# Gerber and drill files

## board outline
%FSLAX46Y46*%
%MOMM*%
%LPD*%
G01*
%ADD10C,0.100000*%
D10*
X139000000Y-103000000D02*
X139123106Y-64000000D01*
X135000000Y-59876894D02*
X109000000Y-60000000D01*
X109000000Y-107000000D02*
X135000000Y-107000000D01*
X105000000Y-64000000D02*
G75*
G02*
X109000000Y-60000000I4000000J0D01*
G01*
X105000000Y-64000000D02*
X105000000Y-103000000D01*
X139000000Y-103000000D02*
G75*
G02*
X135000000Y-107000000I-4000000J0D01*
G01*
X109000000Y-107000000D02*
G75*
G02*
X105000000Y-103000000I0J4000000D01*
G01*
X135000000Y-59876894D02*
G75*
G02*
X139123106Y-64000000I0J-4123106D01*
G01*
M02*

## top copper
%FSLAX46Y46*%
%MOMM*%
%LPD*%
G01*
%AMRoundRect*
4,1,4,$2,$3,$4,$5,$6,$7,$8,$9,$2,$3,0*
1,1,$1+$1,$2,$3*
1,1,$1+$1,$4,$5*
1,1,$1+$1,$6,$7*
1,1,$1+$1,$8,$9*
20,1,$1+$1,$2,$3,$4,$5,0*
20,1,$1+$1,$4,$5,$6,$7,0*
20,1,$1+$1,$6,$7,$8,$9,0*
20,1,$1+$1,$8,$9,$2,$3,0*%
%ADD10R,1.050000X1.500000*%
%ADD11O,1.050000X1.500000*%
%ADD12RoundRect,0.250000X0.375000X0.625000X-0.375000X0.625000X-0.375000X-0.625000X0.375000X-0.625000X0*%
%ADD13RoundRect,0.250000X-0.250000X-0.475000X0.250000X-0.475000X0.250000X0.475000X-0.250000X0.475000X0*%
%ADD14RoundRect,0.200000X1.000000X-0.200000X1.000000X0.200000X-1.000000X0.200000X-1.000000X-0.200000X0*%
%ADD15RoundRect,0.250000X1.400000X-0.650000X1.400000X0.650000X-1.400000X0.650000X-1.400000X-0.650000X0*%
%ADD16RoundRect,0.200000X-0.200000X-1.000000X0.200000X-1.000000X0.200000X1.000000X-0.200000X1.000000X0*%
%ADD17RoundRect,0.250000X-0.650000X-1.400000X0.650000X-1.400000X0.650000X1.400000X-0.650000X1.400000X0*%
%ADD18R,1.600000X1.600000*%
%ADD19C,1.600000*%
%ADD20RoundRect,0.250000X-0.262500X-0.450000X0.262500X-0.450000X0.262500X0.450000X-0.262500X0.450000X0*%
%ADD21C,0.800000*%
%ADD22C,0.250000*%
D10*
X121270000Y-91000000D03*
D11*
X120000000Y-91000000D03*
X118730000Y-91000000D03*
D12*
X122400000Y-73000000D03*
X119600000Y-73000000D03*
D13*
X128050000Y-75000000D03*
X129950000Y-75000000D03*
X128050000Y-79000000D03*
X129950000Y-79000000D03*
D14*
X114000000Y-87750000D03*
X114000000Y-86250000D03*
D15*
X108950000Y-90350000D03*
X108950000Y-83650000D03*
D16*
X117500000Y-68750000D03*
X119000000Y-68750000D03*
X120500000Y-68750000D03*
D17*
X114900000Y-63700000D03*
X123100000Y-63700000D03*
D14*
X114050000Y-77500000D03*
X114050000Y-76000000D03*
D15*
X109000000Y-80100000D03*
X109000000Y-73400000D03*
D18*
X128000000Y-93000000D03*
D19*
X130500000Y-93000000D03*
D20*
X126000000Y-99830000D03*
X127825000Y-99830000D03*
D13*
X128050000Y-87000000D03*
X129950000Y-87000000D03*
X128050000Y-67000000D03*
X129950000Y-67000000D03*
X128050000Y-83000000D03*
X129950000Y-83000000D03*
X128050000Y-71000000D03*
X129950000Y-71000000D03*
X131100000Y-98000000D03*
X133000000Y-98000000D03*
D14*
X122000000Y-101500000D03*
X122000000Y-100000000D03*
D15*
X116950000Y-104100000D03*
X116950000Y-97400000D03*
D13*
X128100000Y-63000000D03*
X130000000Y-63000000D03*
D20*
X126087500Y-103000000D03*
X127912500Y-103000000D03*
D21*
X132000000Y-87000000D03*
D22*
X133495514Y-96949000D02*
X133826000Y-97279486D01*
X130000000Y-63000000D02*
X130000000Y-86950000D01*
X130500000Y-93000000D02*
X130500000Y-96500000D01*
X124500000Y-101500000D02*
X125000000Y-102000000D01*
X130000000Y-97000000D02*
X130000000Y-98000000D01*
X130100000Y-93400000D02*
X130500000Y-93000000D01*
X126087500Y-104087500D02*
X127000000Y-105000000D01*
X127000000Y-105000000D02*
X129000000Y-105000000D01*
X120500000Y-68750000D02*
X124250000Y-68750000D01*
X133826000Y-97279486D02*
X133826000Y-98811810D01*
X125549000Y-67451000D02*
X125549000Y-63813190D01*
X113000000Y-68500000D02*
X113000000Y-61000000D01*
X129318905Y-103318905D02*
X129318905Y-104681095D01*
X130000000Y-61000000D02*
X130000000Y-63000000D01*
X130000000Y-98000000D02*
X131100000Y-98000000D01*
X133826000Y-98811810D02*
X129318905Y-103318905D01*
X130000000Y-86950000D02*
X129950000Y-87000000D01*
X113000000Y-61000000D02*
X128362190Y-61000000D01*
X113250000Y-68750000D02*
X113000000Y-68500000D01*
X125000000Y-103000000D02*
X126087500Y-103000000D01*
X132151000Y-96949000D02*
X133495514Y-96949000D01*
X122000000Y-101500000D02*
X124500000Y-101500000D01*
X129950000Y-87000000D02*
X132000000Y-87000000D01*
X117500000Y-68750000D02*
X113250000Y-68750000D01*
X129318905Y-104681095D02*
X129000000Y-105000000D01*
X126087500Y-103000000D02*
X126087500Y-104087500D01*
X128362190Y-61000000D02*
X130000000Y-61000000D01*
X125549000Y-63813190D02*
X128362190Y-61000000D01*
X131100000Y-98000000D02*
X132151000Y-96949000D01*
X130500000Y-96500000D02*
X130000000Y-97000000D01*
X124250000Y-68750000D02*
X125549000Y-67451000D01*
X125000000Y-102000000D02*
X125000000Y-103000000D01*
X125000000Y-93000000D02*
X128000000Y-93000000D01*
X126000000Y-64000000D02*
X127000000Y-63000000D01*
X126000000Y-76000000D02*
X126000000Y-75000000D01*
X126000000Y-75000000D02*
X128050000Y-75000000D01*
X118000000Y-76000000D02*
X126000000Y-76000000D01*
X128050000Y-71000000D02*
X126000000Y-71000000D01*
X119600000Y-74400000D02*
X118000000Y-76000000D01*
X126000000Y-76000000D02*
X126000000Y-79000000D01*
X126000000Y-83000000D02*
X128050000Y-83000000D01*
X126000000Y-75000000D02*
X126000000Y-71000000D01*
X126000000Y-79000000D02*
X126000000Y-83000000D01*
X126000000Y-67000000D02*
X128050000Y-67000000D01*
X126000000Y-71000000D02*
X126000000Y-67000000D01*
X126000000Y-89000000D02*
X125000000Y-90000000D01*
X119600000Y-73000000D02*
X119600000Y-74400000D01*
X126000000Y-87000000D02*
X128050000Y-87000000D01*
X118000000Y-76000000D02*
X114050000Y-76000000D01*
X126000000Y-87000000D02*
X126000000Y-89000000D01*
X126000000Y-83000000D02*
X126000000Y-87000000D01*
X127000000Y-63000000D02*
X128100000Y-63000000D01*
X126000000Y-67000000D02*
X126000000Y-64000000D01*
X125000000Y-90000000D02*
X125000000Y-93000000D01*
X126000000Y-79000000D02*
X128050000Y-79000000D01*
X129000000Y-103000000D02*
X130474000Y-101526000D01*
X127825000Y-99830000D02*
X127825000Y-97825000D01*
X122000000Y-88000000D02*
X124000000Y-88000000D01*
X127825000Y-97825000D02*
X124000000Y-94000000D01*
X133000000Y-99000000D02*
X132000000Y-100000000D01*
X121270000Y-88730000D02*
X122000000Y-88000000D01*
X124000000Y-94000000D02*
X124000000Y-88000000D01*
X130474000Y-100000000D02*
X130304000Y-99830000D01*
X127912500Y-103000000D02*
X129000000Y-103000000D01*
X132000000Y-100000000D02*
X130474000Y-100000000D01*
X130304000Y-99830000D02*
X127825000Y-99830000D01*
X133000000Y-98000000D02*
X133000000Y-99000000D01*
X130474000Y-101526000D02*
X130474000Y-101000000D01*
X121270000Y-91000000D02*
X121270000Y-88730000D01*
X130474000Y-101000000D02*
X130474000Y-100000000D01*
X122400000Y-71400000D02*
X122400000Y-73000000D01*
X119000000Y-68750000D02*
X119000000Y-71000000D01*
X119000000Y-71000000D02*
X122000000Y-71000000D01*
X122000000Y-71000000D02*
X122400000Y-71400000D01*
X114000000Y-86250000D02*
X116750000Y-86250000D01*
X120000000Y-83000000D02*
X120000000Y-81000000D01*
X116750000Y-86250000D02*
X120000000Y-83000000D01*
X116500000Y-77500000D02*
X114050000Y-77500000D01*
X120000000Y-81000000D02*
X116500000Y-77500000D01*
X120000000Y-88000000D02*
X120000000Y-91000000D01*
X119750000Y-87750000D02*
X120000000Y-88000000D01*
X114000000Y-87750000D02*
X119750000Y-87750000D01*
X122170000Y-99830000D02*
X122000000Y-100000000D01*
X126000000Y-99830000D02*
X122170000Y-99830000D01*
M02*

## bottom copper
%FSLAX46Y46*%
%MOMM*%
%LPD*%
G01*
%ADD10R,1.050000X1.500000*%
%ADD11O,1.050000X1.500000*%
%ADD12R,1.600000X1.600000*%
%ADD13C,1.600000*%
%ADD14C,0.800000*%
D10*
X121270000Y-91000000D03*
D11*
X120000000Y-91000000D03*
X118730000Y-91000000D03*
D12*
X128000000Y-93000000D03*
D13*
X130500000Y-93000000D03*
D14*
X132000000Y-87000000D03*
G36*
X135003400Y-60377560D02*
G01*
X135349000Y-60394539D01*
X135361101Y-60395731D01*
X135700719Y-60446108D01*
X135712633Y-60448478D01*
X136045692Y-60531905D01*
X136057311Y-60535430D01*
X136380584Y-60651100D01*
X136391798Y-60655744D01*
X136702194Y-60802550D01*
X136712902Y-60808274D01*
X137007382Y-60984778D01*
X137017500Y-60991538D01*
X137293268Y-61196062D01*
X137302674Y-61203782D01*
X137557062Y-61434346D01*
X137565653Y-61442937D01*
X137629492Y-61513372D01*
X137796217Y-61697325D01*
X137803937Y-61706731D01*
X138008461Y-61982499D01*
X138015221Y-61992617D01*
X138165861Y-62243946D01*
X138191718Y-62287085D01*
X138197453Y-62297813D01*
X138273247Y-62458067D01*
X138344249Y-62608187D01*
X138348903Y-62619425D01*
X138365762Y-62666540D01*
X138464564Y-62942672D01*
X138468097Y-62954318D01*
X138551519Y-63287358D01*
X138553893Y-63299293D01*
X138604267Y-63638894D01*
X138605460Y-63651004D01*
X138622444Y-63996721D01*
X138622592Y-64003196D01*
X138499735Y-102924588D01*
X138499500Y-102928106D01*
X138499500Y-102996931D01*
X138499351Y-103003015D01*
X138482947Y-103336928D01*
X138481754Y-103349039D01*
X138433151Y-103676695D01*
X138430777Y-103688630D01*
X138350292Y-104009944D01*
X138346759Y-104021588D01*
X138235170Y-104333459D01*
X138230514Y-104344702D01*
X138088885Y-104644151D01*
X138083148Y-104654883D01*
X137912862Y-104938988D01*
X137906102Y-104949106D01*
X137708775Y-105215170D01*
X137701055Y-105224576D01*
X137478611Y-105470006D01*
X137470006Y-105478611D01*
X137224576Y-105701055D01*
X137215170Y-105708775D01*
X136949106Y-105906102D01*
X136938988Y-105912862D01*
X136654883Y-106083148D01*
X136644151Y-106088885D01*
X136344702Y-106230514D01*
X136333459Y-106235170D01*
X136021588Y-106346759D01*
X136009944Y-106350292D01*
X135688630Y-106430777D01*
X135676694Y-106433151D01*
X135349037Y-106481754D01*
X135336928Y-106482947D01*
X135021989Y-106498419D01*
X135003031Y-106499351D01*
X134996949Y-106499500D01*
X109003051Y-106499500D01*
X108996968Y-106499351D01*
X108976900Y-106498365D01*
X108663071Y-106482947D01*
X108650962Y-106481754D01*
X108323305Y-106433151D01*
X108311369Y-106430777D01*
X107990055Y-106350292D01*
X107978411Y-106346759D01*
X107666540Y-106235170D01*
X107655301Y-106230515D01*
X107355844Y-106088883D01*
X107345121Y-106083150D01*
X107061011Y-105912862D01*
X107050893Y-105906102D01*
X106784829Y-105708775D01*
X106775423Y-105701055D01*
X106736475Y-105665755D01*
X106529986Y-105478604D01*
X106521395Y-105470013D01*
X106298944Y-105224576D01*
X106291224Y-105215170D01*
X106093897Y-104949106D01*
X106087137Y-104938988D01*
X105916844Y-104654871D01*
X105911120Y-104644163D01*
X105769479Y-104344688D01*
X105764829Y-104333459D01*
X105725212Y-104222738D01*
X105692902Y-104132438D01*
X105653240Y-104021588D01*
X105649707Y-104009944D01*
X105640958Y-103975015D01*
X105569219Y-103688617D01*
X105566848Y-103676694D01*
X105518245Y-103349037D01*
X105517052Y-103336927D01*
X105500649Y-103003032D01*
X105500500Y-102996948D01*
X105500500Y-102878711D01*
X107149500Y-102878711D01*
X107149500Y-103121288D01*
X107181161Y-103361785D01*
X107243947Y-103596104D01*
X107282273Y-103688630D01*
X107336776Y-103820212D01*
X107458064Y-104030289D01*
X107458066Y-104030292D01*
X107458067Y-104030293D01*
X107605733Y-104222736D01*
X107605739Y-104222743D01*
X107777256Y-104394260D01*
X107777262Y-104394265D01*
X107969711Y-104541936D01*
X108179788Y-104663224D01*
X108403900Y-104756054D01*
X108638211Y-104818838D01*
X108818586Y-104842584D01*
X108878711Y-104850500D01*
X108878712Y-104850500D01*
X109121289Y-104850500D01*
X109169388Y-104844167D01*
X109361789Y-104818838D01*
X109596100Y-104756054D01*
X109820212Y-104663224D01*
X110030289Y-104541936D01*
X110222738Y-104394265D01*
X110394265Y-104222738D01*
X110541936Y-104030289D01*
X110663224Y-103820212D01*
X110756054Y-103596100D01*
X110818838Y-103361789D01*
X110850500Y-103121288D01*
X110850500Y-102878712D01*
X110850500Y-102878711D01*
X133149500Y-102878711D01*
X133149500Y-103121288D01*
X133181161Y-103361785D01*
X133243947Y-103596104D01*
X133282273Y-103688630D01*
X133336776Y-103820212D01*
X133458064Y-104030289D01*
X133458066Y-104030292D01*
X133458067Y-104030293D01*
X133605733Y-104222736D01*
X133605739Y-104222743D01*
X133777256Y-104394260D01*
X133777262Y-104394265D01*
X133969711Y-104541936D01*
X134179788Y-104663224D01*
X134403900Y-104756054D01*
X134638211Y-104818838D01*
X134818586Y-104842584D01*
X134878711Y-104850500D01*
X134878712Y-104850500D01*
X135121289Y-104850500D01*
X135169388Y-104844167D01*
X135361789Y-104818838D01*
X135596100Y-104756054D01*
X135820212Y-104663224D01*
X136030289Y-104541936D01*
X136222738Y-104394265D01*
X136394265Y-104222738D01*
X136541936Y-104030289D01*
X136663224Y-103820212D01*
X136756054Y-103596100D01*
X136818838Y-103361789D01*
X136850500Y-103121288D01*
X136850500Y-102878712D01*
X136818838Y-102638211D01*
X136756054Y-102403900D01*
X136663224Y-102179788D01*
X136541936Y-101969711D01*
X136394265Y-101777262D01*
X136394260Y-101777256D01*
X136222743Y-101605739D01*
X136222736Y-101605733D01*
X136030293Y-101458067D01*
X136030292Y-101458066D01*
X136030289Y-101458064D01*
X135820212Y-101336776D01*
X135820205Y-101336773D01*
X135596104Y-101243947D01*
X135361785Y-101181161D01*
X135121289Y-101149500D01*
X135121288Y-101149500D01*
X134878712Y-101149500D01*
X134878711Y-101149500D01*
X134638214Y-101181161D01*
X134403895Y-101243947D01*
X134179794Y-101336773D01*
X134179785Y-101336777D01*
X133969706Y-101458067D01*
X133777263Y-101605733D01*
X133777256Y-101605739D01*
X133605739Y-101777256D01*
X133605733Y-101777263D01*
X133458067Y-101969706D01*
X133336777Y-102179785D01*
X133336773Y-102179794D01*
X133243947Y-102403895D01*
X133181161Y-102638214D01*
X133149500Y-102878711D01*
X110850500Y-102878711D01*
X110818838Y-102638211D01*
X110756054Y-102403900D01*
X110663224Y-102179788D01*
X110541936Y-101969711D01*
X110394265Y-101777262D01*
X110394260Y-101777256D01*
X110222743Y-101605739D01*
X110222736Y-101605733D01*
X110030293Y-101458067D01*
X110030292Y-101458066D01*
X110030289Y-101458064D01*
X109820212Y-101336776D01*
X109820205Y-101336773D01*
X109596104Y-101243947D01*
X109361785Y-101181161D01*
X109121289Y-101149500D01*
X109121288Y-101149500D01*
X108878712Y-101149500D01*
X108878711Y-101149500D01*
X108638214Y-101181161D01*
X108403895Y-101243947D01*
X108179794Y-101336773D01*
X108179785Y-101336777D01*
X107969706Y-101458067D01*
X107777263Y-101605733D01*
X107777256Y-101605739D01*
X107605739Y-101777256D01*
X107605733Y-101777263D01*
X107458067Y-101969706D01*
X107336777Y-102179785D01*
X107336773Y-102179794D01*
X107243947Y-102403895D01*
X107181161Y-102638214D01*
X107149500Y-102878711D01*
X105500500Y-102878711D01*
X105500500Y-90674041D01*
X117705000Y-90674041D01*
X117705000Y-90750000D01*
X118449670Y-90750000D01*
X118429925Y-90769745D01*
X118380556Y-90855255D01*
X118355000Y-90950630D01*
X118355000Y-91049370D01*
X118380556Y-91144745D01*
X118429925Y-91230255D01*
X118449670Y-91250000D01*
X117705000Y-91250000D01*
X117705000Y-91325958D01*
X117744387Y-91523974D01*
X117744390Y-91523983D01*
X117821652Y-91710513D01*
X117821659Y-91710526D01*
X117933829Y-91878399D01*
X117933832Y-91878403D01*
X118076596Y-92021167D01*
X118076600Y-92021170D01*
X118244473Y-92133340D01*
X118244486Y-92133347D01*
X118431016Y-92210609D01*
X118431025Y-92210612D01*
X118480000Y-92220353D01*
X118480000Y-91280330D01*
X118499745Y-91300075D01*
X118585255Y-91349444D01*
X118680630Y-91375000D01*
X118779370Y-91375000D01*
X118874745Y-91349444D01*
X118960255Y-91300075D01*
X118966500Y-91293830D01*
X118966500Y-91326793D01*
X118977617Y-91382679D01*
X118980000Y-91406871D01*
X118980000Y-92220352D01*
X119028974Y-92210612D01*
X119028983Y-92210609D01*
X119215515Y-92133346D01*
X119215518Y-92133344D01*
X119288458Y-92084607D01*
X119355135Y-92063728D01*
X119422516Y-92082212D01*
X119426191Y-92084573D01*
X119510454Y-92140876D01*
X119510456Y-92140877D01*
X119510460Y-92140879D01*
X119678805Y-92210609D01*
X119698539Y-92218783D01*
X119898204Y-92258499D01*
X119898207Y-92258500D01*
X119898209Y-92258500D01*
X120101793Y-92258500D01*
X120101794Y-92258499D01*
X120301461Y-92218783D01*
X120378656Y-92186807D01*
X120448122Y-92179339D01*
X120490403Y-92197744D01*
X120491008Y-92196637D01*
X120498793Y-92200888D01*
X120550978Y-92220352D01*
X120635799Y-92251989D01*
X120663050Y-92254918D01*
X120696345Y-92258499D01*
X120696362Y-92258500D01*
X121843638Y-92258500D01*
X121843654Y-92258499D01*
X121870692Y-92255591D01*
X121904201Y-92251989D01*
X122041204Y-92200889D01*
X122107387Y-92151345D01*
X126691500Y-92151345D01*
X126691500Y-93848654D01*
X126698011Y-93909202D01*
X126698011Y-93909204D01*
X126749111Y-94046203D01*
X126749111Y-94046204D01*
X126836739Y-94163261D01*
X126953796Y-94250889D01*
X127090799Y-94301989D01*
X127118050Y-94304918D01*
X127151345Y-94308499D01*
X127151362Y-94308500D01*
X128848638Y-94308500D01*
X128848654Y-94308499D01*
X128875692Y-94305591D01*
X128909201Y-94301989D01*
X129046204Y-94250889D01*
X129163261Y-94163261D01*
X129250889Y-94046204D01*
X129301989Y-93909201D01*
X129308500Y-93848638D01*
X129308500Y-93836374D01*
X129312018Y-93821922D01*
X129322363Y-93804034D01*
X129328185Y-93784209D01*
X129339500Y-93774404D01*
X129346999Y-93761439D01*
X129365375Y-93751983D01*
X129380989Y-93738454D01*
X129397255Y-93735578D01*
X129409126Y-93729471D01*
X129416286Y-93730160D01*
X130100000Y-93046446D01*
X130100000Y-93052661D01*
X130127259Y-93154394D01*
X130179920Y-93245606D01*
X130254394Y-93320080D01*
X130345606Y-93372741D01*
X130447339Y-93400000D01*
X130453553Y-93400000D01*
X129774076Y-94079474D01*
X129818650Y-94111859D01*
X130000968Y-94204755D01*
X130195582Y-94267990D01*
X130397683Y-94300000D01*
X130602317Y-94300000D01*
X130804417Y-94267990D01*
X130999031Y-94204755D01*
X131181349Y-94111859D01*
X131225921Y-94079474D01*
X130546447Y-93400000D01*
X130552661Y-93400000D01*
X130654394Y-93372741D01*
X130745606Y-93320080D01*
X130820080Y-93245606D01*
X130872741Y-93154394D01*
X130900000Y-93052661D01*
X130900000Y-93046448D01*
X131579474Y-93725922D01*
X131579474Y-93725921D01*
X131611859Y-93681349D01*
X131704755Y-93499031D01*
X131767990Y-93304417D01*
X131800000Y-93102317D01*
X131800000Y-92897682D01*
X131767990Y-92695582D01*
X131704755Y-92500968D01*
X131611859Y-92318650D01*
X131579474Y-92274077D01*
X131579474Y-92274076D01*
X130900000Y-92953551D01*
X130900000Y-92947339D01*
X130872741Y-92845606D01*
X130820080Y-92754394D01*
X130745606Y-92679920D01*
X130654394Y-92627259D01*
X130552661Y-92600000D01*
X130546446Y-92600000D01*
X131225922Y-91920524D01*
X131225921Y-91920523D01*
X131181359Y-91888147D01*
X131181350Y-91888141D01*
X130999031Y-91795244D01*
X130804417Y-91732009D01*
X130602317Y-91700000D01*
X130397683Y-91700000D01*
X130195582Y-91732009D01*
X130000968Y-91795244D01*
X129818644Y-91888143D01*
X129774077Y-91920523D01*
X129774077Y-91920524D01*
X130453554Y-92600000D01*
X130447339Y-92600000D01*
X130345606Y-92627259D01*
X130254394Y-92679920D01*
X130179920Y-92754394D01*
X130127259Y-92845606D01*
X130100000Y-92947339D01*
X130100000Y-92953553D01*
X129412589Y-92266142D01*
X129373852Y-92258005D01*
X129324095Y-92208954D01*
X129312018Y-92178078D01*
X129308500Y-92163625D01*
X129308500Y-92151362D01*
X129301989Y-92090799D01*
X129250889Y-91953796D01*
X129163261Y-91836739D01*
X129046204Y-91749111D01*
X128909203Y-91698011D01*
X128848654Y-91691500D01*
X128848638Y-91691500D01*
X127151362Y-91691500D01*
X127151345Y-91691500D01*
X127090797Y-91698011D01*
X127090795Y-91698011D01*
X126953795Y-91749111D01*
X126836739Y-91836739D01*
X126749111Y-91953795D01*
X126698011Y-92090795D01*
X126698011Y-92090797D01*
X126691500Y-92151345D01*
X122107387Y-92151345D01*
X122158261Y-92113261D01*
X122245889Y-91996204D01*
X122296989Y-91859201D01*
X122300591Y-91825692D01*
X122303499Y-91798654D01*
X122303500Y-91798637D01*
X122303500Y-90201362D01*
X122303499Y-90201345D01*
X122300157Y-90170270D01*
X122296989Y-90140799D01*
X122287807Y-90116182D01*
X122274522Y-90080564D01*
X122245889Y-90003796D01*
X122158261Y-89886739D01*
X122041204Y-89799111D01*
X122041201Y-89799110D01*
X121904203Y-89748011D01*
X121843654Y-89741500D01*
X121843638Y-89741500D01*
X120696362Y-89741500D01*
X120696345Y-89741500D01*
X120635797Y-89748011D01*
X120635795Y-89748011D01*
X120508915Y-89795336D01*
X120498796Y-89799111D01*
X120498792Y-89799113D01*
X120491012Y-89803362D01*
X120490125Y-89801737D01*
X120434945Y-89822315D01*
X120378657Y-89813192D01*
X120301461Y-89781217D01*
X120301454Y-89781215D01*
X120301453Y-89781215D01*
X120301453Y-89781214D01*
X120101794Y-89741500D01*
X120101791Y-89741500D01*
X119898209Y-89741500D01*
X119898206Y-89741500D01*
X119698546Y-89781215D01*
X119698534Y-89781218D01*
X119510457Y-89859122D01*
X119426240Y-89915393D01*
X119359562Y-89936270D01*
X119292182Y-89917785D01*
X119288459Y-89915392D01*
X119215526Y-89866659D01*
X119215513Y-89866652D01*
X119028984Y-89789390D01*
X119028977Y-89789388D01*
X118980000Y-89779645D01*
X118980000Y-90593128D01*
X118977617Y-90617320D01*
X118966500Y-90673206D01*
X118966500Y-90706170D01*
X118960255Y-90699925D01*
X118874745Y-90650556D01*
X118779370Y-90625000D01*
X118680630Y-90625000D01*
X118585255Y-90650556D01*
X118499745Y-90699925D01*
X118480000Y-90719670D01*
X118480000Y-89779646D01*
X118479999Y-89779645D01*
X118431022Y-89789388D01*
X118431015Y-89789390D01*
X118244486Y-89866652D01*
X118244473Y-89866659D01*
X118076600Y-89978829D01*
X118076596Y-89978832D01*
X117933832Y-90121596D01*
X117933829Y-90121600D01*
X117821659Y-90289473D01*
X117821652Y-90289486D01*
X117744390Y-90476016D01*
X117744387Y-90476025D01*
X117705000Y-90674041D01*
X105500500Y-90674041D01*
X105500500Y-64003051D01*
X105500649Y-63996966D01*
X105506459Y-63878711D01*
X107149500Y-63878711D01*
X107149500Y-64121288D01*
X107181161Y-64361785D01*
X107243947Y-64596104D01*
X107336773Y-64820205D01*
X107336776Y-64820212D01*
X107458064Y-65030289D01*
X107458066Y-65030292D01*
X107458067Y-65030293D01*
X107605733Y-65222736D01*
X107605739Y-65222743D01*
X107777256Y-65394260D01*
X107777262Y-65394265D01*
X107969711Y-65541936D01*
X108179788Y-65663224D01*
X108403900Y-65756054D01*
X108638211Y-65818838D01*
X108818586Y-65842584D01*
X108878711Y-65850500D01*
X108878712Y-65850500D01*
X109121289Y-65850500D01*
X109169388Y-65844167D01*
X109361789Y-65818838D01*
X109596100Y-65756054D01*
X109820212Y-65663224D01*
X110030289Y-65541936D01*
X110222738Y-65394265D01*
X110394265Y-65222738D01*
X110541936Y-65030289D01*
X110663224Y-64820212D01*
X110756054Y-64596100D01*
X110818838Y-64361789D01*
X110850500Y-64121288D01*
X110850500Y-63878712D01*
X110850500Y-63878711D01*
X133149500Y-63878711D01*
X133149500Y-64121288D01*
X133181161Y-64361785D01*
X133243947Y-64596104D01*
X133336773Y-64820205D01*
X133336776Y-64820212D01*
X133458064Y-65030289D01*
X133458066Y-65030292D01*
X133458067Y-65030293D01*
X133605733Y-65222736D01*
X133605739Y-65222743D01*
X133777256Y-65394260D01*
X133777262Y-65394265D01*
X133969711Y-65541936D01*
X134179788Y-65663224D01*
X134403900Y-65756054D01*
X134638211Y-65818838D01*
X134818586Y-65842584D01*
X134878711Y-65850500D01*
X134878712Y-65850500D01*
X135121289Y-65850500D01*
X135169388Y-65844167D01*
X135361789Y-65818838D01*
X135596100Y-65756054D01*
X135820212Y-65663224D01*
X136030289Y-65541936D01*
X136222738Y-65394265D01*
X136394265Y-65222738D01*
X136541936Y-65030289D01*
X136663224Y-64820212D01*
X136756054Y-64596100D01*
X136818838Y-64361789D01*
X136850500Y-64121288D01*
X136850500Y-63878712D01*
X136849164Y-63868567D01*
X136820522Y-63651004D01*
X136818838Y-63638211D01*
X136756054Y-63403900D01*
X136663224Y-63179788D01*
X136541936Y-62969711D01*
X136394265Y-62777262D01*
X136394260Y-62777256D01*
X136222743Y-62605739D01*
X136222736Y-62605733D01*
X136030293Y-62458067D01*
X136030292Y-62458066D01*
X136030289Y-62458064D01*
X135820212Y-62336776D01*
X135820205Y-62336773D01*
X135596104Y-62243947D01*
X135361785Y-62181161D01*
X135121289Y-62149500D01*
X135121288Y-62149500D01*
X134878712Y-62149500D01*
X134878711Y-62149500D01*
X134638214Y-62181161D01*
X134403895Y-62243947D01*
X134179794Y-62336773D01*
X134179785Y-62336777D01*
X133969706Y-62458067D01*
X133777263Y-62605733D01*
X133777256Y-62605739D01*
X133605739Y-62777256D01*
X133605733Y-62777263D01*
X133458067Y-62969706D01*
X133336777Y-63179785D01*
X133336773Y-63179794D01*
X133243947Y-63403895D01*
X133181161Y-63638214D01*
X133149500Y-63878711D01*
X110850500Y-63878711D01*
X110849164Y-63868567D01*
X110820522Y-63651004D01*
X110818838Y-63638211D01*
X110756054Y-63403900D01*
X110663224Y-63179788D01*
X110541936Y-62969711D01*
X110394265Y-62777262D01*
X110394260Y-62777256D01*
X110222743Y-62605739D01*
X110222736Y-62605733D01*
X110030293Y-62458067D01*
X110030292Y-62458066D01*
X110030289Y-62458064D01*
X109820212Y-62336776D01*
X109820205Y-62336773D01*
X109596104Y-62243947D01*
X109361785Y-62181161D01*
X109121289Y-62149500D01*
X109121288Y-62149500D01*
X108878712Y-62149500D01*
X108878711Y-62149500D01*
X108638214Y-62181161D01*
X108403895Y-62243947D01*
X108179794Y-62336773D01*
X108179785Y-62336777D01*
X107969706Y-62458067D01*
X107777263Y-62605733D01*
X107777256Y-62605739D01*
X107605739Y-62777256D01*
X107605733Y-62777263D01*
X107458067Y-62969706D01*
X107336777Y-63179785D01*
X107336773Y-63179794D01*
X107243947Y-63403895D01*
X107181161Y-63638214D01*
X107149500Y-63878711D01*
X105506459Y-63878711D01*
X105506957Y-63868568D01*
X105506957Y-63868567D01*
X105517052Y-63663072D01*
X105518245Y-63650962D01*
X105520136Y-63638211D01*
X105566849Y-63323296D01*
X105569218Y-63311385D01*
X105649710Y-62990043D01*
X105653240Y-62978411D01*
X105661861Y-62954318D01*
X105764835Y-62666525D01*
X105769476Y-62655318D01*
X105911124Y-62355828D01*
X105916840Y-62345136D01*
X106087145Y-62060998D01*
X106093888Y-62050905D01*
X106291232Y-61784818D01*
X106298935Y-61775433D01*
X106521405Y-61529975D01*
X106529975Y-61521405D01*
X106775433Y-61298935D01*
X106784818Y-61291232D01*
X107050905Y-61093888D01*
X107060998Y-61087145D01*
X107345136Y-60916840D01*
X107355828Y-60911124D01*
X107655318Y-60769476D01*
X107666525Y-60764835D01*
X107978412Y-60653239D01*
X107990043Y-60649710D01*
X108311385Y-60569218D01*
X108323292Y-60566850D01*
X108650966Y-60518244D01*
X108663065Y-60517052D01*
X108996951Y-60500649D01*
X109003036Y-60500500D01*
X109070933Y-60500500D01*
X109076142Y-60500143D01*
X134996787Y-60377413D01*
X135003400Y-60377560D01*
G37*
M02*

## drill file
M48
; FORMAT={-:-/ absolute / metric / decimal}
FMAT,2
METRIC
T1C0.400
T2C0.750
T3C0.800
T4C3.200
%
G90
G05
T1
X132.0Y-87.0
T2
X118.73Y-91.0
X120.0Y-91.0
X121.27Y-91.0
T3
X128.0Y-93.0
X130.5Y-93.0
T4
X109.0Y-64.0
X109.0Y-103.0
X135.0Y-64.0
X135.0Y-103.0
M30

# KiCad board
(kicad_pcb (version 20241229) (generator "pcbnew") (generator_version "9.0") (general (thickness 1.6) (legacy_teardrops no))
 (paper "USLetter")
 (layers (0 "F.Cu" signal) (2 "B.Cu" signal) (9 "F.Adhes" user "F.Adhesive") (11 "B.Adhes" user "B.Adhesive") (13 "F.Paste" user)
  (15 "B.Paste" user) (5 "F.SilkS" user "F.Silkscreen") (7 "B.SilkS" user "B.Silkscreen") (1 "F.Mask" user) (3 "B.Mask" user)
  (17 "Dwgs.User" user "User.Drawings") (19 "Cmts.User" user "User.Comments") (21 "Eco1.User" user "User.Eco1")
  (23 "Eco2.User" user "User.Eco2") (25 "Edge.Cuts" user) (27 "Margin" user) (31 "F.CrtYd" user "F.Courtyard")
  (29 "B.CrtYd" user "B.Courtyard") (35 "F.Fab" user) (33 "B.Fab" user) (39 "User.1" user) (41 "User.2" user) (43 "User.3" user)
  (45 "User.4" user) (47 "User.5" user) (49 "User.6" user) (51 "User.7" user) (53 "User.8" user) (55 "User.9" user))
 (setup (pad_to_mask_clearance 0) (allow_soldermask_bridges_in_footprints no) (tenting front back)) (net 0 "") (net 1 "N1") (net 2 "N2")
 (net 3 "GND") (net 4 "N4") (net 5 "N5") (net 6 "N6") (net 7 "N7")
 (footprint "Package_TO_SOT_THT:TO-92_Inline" (layer "F.Cu") (at 121.27 91 180)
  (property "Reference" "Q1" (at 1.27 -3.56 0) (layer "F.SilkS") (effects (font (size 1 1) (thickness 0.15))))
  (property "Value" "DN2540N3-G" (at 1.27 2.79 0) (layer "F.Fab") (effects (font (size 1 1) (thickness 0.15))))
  (pad "1" thru_hole rect (at 0 0 180) (size 1.05 1.5) (drill 0.75) (layers "*.Cu" "*.Mask") (remove_unused_layers no) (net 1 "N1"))
  (pad "2" thru_hole oval (at 1.27 0 180) (size 1.05 1.5) (drill 0.75) (layers "*.Cu" "*.Mask") (remove_unused_layers no) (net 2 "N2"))
  (pad "3" thru_hole oval (at 2.54 0 180) (size 1.05 1.5) (drill 0.75) (layers "*.Cu" "*.Mask") (remove_unused_layers no) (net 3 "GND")))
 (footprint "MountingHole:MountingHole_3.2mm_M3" (layer "F.Cu") (at 135 64)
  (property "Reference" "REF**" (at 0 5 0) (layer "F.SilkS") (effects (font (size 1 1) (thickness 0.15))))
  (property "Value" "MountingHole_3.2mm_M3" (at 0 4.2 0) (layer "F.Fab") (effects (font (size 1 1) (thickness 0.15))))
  (pad "" np_thru_hole circle (at 0 0) (size 3.2 3.2) (drill 3.2) (layers "*.Cu" "*.Mask")))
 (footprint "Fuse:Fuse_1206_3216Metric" (layer "F.Cu") (at 121 73 180)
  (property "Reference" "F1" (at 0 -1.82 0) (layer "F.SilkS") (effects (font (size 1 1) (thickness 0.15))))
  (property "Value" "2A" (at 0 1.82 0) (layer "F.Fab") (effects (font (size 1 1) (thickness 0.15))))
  (pad "1" smd roundrect (at -1.4 0 180) (size 1.25 1.75) (layers "F.Cu" "F.Mask" "F.Paste") (roundrect_rratio 0.2) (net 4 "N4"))
  (pad "2" smd roundrect (at 1.4 0 180) (size 1.25 1.75) (layers "F.Cu" "F.Mask" "F.Paste") (roundrect_rratio 0.2) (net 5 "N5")))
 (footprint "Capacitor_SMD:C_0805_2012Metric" (layer "F.Cu") (at 129 75)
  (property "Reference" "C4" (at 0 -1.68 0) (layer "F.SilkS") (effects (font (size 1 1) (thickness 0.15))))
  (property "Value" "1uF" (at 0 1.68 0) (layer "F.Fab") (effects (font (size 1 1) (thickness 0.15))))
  (pad "1" smd roundrect (at -0.95 0) (size 1 1.45) (layers "F.Cu" "F.Mask" "F.Paste") (roundrect_rratio 0.25) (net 5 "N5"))
  (pad "2" smd roundrect (at 0.95 0) (size 1 1.45) (layers "F.Cu" "F.Mask" "F.Paste") (roundrect_rratio 0.25) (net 3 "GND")))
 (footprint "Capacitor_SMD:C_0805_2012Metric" (layer "F.Cu") (at 129 79)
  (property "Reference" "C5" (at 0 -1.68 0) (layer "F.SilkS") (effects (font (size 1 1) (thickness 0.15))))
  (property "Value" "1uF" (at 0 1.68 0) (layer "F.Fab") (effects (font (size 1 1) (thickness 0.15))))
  (pad "1" smd roundrect (at -0.95 0) (size 1 1.45) (layers "F.Cu" "F.Mask" "F.Paste") (roundrect_rratio 0.25) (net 5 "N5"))
  (pad "2" smd roundrect (at 0.95 0) (size 1 1.45) (layers "F.Cu" "F.Mask" "F.Paste") (roundrect_rratio 0.25) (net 3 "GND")))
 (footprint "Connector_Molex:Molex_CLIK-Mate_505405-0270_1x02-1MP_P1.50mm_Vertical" (layer "F.Cu") (at 111.25 87 90)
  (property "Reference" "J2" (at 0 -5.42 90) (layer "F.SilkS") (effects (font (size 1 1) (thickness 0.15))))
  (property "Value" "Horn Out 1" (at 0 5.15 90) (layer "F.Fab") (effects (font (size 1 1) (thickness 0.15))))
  (pad "1" smd roundrect (at -0.75 2.75 90) (size 0.8 2.4) (layers "F.Cu" "F.Mask" "F.Paste") (roundrect_rratio 0.25) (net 2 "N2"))
  (pad "2" smd roundrect (at 0.75 2.75 90) (size 0.8 2.4) (layers "F.Cu" "F.Mask" "F.Paste") (roundrect_rratio 0.25) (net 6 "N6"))
  (pad "MP" smd roundrect (at -3.35 -2.3 90) (size 1.8 3.3) (layers "F.Cu" "F.Mask" "F.Paste") (roundrect_rratio 0.138889))
  (pad "MP" smd roundrect (at 3.35 -2.3 90) (size 1.8 3.3) (layers "F.Cu" "F.Mask" "F.Paste") (roundrect_rratio 0.138889)))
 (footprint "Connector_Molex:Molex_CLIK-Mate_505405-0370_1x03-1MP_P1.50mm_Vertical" (layer "F.Cu") (at 119 66)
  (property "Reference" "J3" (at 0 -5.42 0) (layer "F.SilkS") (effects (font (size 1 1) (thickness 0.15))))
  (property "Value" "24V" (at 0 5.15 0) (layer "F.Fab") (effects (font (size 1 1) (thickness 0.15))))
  (pad "1" smd roundrect (at -1.5 2.75) (size 0.8 2.4) (layers "F.Cu" "F.Mask" "F.Paste") (roundrect_rratio 0.25) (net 3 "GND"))
  (pad "2" smd roundrect (at 0 2.75) (size 0.8 2.4) (layers "F.Cu" "F.Mask" "F.Paste") (roundrect_rratio 0.25) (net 4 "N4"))
  (pad "3" smd roundrect (at 1.5 2.75) (size 0.8 2.4) (layers "F.Cu" "F.Mask" "F.Paste") (roundrect_rratio 0.25) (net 3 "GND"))
  (pad "MP" smd roundrect (at -4.1 -2.3) (size 1.8 3.3) (layers "F.Cu" "F.Mask" "F.Paste") (roundrect_rratio 0.138889))
  (pad "MP" smd roundrect (at 4.1 -2.3) (size 1.8 3.3) (layers "F.Cu" "F.Mask" "F.Paste") (roundrect_rratio 0.138889)))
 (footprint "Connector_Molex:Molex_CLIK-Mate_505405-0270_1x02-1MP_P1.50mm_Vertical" (layer "F.Cu") (at 111.3 76.75 90)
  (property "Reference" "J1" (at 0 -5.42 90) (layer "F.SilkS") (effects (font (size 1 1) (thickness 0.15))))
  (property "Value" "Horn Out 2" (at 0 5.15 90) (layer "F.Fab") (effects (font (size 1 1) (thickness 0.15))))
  (pad "1" smd roundrect (at -0.75 2.75 90) (size 0.8 2.4) (layers "F.Cu" "F.Mask" "F.Paste") (roundrect_rratio 0.25) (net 6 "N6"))
  (pad "2" smd roundrect (at 0.75 2.75 90) (size 0.8 2.4) (layers "F.Cu" "F.Mask" "F.Paste") (roundrect_rratio 0.25) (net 5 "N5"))
  (pad "MP" smd roundrect (at -3.35 -2.3 90) (size 1.8 3.3) (layers "F.Cu" "F.Mask" "F.Paste") (roundrect_rratio 0.138889))
  (pad "MP" smd roundrect (at 3.35 -2.3 90) (size 1.8 3.3) (layers "F.Cu" "F.Mask" "F.Paste") (roundrect_rratio 0.138889)))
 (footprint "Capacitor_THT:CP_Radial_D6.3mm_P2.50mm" (layer "F.Cu") (at 128 93)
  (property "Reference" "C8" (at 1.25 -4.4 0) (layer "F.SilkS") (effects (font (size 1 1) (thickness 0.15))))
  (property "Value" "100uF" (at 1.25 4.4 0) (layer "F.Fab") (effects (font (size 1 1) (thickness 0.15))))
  (pad "1" thru_hole rect (at 0 0) (size 1.6 1.6) (drill 0.8) (layers "*.Cu" "*.Mask") (remove_unused_layers no) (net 5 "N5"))
  (pad "2" thru_hole circle (at 2.5 0) (size 1.6 1.6) (drill 0.8) (layers "*.Cu" "*.Mask") (remove_unused_layers no) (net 3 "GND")))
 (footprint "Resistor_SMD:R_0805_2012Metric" (layer "F.Cu") (at 126.9125 99.83)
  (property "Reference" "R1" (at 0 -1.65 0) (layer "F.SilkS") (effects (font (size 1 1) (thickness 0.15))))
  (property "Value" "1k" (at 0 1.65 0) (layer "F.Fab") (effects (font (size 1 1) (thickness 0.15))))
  (pad "1" smd roundrect (at -0.9125 0) (size 1.025 1.4) (layers "F.Cu" "F.Mask" "F.Paste") (roundrect_rratio 0.243902) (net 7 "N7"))
  (pad "2" smd roundrect (at 0.9125 0) (size 1.025 1.4) (layers "F.Cu" "F.Mask" "F.Paste") (roundrect_rratio 0.243902) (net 1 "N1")))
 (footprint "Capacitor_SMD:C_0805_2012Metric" (layer "F.Cu") (at 129 87)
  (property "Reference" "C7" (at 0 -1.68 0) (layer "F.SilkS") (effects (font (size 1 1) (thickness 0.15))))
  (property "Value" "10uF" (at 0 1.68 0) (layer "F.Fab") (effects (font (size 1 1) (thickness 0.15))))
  (pad "1" smd roundrect (at -0.95 0) (size 1 1.45) (layers "F.Cu" "F.Mask" "F.Paste") (roundrect_rratio 0.25) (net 5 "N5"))
  (pad "2" smd roundrect (at 0.95 0) (size 1 1.45) (layers "F.Cu" "F.Mask" "F.Paste") (roundrect_rratio 0.25) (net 3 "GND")))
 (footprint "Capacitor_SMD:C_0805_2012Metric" (layer "F.Cu") (at 129 67)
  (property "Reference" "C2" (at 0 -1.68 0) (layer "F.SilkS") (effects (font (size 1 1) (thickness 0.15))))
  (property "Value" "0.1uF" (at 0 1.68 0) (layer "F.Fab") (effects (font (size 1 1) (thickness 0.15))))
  (pad "1" smd roundrect (at -0.95 0) (size 1 1.45) (layers "F.Cu" "F.Mask" "F.Paste") (roundrect_rratio 0.25) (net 5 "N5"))
  (pad "2" smd roundrect (at 0.95 0) (size 1 1.45) (layers "F.Cu" "F.Mask" "F.Paste") (roundrect_rratio 0.25) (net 3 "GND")))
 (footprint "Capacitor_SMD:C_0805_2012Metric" (layer "F.Cu") (at 129 83)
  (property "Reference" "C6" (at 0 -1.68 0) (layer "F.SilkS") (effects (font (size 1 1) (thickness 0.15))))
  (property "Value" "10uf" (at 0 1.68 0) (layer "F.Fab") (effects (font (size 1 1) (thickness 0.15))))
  (pad "1" smd roundrect (at -0.95 0) (size 1 1.45) (layers "F.Cu" "F.Mask" "F.Paste") (roundrect_rratio 0.25) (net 5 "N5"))
  (pad "2" smd roundrect (at 0.95 0) (size 1 1.45) (layers "F.Cu" "F.Mask" "F.Paste") (roundrect_rratio 0.25) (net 3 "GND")))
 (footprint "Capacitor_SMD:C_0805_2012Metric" (layer "F.Cu") (at 129 71)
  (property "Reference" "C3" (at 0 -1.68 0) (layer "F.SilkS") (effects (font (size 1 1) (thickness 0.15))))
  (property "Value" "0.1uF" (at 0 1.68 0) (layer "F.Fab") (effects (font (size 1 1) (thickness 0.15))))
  (pad "1" smd roundrect (at -0.95 0) (size 1 1.45) (layers "F.Cu" "F.Mask" "F.Paste") (roundrect_rratio 0.25) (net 5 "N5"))
  (pad "2" smd roundrect (at 0.95 0) (size 1 1.45) (layers "F.Cu" "F.Mask" "F.Paste") (roundrect_rratio 0.25) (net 3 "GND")))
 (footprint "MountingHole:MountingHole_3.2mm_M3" (layer "F.Cu") (at 109 64)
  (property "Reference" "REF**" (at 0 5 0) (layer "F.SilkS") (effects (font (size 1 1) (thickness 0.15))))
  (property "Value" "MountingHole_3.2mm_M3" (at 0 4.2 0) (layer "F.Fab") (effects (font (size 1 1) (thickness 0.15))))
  (pad "" np_thru_hole circle (at 0 0) (size 3.2 3.2) (drill 3.2) (layers "*.Cu" "*.Mask")))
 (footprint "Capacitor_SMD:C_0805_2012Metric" (layer "F.Cu") (at 132.05 98)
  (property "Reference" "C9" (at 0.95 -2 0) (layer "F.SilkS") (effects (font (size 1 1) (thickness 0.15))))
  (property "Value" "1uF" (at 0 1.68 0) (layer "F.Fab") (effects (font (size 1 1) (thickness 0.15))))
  (pad "1" smd roundrect (at -0.95 0) (size 1 1.45) (layers "F.Cu" "F.Mask" "F.Paste") (roundrect_rratio 0.25) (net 3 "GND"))
  (pad "2" smd roundrect (at 0.95 0) (size 1 1.45) (layers "F.Cu" "F.Mask" "F.Paste") (roundrect_rratio 0.25) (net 1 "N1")))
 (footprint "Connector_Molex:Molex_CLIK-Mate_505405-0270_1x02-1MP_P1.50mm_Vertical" (layer "F.Cu") (at 119.25 100.75 90)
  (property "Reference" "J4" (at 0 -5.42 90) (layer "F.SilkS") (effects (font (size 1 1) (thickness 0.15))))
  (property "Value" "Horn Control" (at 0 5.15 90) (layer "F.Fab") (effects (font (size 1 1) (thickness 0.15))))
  (pad "1" smd roundrect (at -0.75 2.75 90) (size 0.8 2.4) (layers "F.Cu" "F.Mask" "F.Paste") (roundrect_rratio 0.25) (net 3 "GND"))
  (pad "2" smd roundrect (at 0.75 2.75 90) (size 0.8 2.4) (layers "F.Cu" "F.Mask" "F.Paste") (roundrect_rratio 0.25) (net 7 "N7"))
  (pad "MP" smd roundrect (at -3.35 -2.3 90) (size 1.8 3.3) (layers "F.Cu" "F.Mask" "F.Paste") (roundrect_rratio 0.138889))
  (pad "MP" smd roundrect (at 3.35 -2.3 90) (size 1.8 3.3) (layers "F.Cu" "F.Mask" "F.Paste") (roundrect_rratio 0.138889)))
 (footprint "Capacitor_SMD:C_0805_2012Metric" (layer "F.Cu") (at 129.05 63)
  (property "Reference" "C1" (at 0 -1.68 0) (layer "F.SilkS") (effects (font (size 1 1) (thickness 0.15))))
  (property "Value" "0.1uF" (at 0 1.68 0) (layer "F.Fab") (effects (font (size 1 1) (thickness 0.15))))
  (pad "1" smd roundrect (at -0.95 0) (size 1 1.45) (layers "F.Cu" "F.Mask" "F.Paste") (roundrect_rratio 0.25) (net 5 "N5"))
  (pad "2" smd roundrect (at 0.95 0) (size 1 1.45) (layers "F.Cu" "F.Mask" "F.Paste") (roundrect_rratio 0.25) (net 3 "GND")))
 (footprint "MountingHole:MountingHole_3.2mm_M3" (layer "F.Cu") (at 109 103)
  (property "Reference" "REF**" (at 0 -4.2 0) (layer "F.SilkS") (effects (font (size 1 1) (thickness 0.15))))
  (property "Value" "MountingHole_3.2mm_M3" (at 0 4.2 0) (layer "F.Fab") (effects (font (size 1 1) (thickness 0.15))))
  (pad "" np_thru_hole circle (at 0 0) (size 3.2 3.2) (drill 3.2) (layers "*.Cu" "*.Mask")))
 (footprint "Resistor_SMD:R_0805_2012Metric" (layer "F.Cu") (at 127 103)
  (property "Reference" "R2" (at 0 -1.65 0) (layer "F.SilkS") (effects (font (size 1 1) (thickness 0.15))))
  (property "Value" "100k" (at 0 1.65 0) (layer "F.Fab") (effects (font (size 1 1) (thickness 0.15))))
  (pad "1" smd roundrect (at -0.9125 0) (size 1.025 1.4) (layers "F.Cu" "F.Mask" "F.Paste") (roundrect_rratio 0.243902) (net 3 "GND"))
  (pad "2" smd roundrect (at 0.9125 0) (size 1.025 1.4) (layers "F.Cu" "F.Mask" "F.Paste") (roundrect_rratio 0.243902) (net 1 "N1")))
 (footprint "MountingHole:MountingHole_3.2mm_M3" (layer "F.Cu") (at 135 103)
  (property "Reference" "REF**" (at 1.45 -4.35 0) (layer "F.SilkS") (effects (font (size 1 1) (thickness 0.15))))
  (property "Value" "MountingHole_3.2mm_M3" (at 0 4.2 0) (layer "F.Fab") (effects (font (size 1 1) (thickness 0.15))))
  (pad "" np_thru_hole circle (at 0 0) (size 3.2 3.2) (drill 3.2) (layers "*.Cu" "*.Mask")))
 (gr_line (start 139 103) (end 139.123106 64) (stroke (width 0.1) (type default)) (layer "Edge.Cuts"))
 (gr_line (start 135 59.876894) (end 109 60) (stroke (width 0.1) (type default)) (layer "Edge.Cuts"))
 (gr_line (start 109 107) (end 135 107) (stroke (width 0.1) (type default)) (layer "Edge.Cuts"))
 (gr_arc (start 105 64) (mid 106.171573 61.171573) (end 109 60) (stroke (width 0.1) (type default)) (layer "Edge.Cuts"))
 (gr_line (start 105 64) (end 105 103) (stroke (width 0.1) (type default)) (layer "Edge.Cuts"))
 (gr_arc (start 139 103) (mid 137.828427 105.828427) (end 135 107) (stroke (width 0.1) (type default)) (layer "Edge.Cuts"))
 (gr_arc (start 109 107) (mid 106.171573 105.828427) (end 105 103) (stroke (width 0.1) (type default)) (layer "Edge.Cuts"))
 (gr_arc (start 135 59.876894) (mid 137.915476 61.084524) (end 139.123106 64) (stroke (width 0.1) (type default)) (layer "Edge.Cuts"))
 (segment (start 133.495514 96.949) (end 133.826 97.279486) (width 0.25) (layer "F.Cu") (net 3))
 (segment (start 130 63) (end 130 86.95) (width 0.25) (layer "F.Cu") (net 3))
 (segment (start 130.5 93) (end 130.5 96.5) (width 0.25) (layer "F.Cu") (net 3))
 (segment (start 124.5 101.5) (end 125 102) (width 0.25) (layer "F.Cu") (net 3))
 (segment (start 130 97) (end 130 98) (width 0.25) (layer "F.Cu") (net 3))
 (segment (start 130.1 93.4) (end 130.5 93) (width 0.25) (layer "F.Cu") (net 3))
 (segment (start 126.0875 104.0875) (end 127 105) (width 0.25) (layer "F.Cu") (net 3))
 (segment (start 127 105) (end 129 105) (width 0.25) (layer "F.Cu") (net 3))
 (segment (start 120.5 68.75) (end 124.25 68.75) (width 0.25) (layer "F.Cu") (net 3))
 (segment (start 133.826 97.279486) (end 133.826 98.81181) (width 0.25) (layer "F.Cu") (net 3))
 (segment (start 125.549 67.451) (end 125.549 63.81319) (width 0.25) (layer "F.Cu") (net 3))
 (segment (start 113 68.5) (end 113 61) (width 0.25) (layer "F.Cu") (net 3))
 (segment (start 129.318905 103.318905) (end 129.318905 104.681095) (width 0.25) (layer "F.Cu") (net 3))
 (segment (start 130 61) (end 130 63) (width 0.25) (layer "F.Cu") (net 3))
 (segment (start 130 98) (end 131.1 98) (width 0.25) (layer "F.Cu") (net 3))
 (segment (start 133.826 98.81181) (end 129.318905 103.318905) (width 0.25) (layer "F.Cu") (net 3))
 (segment (start 130 86.95) (end 129.95 87) (width 0.25) (layer "F.Cu") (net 3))
 (segment (start 113 61) (end 128.36219 61) (width 0.25) (layer "F.Cu") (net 3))
 (segment (start 113.25 68.75) (end 113 68.5) (width 0.25) (layer "F.Cu") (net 3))
 (segment (start 125 103) (end 126.0875 103) (width 0.25) (layer "F.Cu") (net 3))
 (segment (start 132.151 96.949) (end 133.495514 96.949) (width 0.25) (layer "F.Cu") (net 3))
 (segment (start 122 101.5) (end 124.5 101.5) (width 0.25) (layer "F.Cu") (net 3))
 (segment (start 129.95 87) (end 132 87) (width 0.25) (layer "F.Cu") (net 3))
 (segment (start 117.5 68.75) (end 113.25 68.75) (width 0.25) (layer "F.Cu") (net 3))
 (segment (start 129.318905 104.681095) (end 129 105) (width 0.25) (layer "F.Cu") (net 3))
 (segment (start 126.0875 103) (end 126.0875 104.0875) (width 0.25) (layer "F.Cu") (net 3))
 (segment (start 128.36219 61) (end 130 61) (width 0.25) (layer "F.Cu") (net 3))
 (segment (start 125.549 63.81319) (end 128.36219 61) (width 0.25) (layer "F.Cu") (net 3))
 (segment (start 131.1 98) (end 132.151 96.949) (width 0.25) (layer "F.Cu") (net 3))
 (segment (start 130.5 96.5) (end 130 97) (width 0.25) (layer "F.Cu") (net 3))
 (segment (start 124.25 68.75) (end 125.549 67.451) (width 0.25) (layer "F.Cu") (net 3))
 (segment (start 125 102) (end 125 103) (width 0.25) (layer "F.Cu") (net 3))
 (via (at 132 87) (size 0.8) (drill 0.4) (layers "F.Cu" "B.Cu") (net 3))
 (segment (start 125 93) (end 128 93) (width 0.25) (layer "F.Cu") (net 5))
 (segment (start 126 64) (end 127 63) (width 0.25) (layer "F.Cu") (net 5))
 (segment (start 126 76) (end 126 75) (width 0.25) (layer "F.Cu") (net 5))
 (segment (start 126 75) (end 128.05 75) (width 0.25) (layer "F.Cu") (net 5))
 (segment (start 118 76) (end 126 76) (width 0.25) (layer "F.Cu") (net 5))
 (segment (start 128.05 71) (end 126 71) (width 0.25) (layer "F.Cu") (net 5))
 (segment (start 119.6 74.4) (end 118 76) (width 0.25) (layer "F.Cu") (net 5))
 (segment (start 126 76) (end 126 79) (width 0.25) (layer "F.Cu") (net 5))
 (segment (start 126 83) (end 128.05 83) (width 0.25) (layer "F.Cu") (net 5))
 (segment (start 126 75) (end 126 71) (width 0.25) (layer "F.Cu") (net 5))
 (segment (start 126 79) (end 126 83) (width 0.25) (layer "F.Cu") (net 5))
 (segment (start 126 67) (end 128.05 67) (width 0.25) (layer "F.Cu") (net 5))
 (segment (start 126 71) (end 126 67) (width 0.25) (layer "F.Cu") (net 5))
 (segment (start 126 89) (end 125 90) (width 0.25) (layer "F.Cu") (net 5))
 (segment (start 119.6 73) (end 119.6 74.4) (width 0.25) (layer "F.Cu") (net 5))
 (segment (start 126 87) (end 128.05 87) (width 0.25) (layer "F.Cu") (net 5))
 (segment (start 118 76) (end 114.05 76) (width 0.25) (layer "F.Cu") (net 5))
 (segment (start 126 87) (end 126 89) (width 0.25) (layer "F.Cu") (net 5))
 (segment (start 126 83) (end 126 87) (width 0.25) (layer "F.Cu") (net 5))
 (segment (start 127 63) (end 128.1 63) (width 0.25) (layer "F.Cu") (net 5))
 (segment (start 126 67) (end 126 64) (width 0.25) (layer "F.Cu") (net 5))
 (segment (start 125 90) (end 125 93) (width 0.25) (layer "F.Cu") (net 5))
 (segment (start 126 79) (end 128.05 79) (width 0.25) (layer "F.Cu") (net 5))
 (segment (start 129 103) (end 130.474 101.526) (width 0.25) (layer "F.Cu") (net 1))
 (segment (start 127.825 99.83) (end 127.825 97.825) (width 0.25) (layer "F.Cu") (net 1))
 (segment (start 122 88) (end 124 88) (width 0.25) (layer "F.Cu") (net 1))
 (segment (start 127.825 97.825) (end 124 94) (width 0.25) (layer "F.Cu") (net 1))
 (segment (start 133 99) (end 132 100) (width 0.25) (layer "F.Cu") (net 1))
 (segment (start 121.27 88.73) (end 122 88) (width 0.25) (layer "F.Cu") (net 1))
 (segment (start 124 94) (end 124 88) (width 0.25) (layer "F.Cu") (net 1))
 (segment (start 130.474 100) (end 130.304 99.83) (width 0.25) (layer "F.Cu") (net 1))
 (segment (start 127.9125 103) (end 129 103) (width 0.25) (layer "F.Cu") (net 1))
 (segment (start 132 100) (end 130.474 100) (width 0.25) (layer "F.Cu") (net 1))
 (segment (start 130.304 99.83) (end 127.825 99.83) (width 0.25) (layer "F.Cu") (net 1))
 (segment (start 133 98) (end 133 99) (width 0.25) (layer "F.Cu") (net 1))
 (segment (start 130.474 101.526) (end 130.474 101) (width 0.25) (layer "F.Cu") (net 1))
 (segment (start 121.27 91) (end 121.27 88.73) (width 0.25) (layer "F.Cu") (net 1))
 (segment (start 130.474 101) (end 130.474 100) (width 0.25) (layer "F.Cu") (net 1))
 (segment (start 122.4 71.4) (end 122.4 73) (width 0.25) (layer "F.Cu") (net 4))
 (segment (start 119 68.75) (end 119 71) (width 0.25) (layer "F.Cu") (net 4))
 (segment (start 119 71) (end 122 71) (width 0.25) (layer "F.Cu") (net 4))
 (segment (start 122 71) (end 122.4 71.4) (width 0.25) (layer "F.Cu") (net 4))
 (segment (start 114 86.25) (end 116.75 86.25) (width 0.25) (layer "F.Cu") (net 6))
 (segment (start 120 83) (end 120 81) (width 0.25) (layer "F.Cu") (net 6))
 (segment (start 116.75 86.25) (end 120 83) (width 0.25) (layer "F.Cu") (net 6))
 (segment (start 116.5 77.5) (end 114.05 77.5) (width 0.25) (layer "F.Cu") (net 6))
 (segment (start 120 81) (end 116.5 77.5) (width 0.25) (layer "F.Cu") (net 6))
 (segment (start 120 88) (end 120 91) (width 0.25) (layer "F.Cu") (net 2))
 (segment (start 119.75 87.75) (end 120 88) (width 0.25) (layer "F.Cu") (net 2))
 (segment (start 114 87.75) (end 119.75 87.75) (width 0.25) (layer "F.Cu") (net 2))
 (segment (start 122.17 99.83) (end 122 100) (width 0.25) (layer "F.Cu") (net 7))
 (segment (start 126 99.83) (end 122.17 99.83) (width 0.25) (layer "F.Cu") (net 7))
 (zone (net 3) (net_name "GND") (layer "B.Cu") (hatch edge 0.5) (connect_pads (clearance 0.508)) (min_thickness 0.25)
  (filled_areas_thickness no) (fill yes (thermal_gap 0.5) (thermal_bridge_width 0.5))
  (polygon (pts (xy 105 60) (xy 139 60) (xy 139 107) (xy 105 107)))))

